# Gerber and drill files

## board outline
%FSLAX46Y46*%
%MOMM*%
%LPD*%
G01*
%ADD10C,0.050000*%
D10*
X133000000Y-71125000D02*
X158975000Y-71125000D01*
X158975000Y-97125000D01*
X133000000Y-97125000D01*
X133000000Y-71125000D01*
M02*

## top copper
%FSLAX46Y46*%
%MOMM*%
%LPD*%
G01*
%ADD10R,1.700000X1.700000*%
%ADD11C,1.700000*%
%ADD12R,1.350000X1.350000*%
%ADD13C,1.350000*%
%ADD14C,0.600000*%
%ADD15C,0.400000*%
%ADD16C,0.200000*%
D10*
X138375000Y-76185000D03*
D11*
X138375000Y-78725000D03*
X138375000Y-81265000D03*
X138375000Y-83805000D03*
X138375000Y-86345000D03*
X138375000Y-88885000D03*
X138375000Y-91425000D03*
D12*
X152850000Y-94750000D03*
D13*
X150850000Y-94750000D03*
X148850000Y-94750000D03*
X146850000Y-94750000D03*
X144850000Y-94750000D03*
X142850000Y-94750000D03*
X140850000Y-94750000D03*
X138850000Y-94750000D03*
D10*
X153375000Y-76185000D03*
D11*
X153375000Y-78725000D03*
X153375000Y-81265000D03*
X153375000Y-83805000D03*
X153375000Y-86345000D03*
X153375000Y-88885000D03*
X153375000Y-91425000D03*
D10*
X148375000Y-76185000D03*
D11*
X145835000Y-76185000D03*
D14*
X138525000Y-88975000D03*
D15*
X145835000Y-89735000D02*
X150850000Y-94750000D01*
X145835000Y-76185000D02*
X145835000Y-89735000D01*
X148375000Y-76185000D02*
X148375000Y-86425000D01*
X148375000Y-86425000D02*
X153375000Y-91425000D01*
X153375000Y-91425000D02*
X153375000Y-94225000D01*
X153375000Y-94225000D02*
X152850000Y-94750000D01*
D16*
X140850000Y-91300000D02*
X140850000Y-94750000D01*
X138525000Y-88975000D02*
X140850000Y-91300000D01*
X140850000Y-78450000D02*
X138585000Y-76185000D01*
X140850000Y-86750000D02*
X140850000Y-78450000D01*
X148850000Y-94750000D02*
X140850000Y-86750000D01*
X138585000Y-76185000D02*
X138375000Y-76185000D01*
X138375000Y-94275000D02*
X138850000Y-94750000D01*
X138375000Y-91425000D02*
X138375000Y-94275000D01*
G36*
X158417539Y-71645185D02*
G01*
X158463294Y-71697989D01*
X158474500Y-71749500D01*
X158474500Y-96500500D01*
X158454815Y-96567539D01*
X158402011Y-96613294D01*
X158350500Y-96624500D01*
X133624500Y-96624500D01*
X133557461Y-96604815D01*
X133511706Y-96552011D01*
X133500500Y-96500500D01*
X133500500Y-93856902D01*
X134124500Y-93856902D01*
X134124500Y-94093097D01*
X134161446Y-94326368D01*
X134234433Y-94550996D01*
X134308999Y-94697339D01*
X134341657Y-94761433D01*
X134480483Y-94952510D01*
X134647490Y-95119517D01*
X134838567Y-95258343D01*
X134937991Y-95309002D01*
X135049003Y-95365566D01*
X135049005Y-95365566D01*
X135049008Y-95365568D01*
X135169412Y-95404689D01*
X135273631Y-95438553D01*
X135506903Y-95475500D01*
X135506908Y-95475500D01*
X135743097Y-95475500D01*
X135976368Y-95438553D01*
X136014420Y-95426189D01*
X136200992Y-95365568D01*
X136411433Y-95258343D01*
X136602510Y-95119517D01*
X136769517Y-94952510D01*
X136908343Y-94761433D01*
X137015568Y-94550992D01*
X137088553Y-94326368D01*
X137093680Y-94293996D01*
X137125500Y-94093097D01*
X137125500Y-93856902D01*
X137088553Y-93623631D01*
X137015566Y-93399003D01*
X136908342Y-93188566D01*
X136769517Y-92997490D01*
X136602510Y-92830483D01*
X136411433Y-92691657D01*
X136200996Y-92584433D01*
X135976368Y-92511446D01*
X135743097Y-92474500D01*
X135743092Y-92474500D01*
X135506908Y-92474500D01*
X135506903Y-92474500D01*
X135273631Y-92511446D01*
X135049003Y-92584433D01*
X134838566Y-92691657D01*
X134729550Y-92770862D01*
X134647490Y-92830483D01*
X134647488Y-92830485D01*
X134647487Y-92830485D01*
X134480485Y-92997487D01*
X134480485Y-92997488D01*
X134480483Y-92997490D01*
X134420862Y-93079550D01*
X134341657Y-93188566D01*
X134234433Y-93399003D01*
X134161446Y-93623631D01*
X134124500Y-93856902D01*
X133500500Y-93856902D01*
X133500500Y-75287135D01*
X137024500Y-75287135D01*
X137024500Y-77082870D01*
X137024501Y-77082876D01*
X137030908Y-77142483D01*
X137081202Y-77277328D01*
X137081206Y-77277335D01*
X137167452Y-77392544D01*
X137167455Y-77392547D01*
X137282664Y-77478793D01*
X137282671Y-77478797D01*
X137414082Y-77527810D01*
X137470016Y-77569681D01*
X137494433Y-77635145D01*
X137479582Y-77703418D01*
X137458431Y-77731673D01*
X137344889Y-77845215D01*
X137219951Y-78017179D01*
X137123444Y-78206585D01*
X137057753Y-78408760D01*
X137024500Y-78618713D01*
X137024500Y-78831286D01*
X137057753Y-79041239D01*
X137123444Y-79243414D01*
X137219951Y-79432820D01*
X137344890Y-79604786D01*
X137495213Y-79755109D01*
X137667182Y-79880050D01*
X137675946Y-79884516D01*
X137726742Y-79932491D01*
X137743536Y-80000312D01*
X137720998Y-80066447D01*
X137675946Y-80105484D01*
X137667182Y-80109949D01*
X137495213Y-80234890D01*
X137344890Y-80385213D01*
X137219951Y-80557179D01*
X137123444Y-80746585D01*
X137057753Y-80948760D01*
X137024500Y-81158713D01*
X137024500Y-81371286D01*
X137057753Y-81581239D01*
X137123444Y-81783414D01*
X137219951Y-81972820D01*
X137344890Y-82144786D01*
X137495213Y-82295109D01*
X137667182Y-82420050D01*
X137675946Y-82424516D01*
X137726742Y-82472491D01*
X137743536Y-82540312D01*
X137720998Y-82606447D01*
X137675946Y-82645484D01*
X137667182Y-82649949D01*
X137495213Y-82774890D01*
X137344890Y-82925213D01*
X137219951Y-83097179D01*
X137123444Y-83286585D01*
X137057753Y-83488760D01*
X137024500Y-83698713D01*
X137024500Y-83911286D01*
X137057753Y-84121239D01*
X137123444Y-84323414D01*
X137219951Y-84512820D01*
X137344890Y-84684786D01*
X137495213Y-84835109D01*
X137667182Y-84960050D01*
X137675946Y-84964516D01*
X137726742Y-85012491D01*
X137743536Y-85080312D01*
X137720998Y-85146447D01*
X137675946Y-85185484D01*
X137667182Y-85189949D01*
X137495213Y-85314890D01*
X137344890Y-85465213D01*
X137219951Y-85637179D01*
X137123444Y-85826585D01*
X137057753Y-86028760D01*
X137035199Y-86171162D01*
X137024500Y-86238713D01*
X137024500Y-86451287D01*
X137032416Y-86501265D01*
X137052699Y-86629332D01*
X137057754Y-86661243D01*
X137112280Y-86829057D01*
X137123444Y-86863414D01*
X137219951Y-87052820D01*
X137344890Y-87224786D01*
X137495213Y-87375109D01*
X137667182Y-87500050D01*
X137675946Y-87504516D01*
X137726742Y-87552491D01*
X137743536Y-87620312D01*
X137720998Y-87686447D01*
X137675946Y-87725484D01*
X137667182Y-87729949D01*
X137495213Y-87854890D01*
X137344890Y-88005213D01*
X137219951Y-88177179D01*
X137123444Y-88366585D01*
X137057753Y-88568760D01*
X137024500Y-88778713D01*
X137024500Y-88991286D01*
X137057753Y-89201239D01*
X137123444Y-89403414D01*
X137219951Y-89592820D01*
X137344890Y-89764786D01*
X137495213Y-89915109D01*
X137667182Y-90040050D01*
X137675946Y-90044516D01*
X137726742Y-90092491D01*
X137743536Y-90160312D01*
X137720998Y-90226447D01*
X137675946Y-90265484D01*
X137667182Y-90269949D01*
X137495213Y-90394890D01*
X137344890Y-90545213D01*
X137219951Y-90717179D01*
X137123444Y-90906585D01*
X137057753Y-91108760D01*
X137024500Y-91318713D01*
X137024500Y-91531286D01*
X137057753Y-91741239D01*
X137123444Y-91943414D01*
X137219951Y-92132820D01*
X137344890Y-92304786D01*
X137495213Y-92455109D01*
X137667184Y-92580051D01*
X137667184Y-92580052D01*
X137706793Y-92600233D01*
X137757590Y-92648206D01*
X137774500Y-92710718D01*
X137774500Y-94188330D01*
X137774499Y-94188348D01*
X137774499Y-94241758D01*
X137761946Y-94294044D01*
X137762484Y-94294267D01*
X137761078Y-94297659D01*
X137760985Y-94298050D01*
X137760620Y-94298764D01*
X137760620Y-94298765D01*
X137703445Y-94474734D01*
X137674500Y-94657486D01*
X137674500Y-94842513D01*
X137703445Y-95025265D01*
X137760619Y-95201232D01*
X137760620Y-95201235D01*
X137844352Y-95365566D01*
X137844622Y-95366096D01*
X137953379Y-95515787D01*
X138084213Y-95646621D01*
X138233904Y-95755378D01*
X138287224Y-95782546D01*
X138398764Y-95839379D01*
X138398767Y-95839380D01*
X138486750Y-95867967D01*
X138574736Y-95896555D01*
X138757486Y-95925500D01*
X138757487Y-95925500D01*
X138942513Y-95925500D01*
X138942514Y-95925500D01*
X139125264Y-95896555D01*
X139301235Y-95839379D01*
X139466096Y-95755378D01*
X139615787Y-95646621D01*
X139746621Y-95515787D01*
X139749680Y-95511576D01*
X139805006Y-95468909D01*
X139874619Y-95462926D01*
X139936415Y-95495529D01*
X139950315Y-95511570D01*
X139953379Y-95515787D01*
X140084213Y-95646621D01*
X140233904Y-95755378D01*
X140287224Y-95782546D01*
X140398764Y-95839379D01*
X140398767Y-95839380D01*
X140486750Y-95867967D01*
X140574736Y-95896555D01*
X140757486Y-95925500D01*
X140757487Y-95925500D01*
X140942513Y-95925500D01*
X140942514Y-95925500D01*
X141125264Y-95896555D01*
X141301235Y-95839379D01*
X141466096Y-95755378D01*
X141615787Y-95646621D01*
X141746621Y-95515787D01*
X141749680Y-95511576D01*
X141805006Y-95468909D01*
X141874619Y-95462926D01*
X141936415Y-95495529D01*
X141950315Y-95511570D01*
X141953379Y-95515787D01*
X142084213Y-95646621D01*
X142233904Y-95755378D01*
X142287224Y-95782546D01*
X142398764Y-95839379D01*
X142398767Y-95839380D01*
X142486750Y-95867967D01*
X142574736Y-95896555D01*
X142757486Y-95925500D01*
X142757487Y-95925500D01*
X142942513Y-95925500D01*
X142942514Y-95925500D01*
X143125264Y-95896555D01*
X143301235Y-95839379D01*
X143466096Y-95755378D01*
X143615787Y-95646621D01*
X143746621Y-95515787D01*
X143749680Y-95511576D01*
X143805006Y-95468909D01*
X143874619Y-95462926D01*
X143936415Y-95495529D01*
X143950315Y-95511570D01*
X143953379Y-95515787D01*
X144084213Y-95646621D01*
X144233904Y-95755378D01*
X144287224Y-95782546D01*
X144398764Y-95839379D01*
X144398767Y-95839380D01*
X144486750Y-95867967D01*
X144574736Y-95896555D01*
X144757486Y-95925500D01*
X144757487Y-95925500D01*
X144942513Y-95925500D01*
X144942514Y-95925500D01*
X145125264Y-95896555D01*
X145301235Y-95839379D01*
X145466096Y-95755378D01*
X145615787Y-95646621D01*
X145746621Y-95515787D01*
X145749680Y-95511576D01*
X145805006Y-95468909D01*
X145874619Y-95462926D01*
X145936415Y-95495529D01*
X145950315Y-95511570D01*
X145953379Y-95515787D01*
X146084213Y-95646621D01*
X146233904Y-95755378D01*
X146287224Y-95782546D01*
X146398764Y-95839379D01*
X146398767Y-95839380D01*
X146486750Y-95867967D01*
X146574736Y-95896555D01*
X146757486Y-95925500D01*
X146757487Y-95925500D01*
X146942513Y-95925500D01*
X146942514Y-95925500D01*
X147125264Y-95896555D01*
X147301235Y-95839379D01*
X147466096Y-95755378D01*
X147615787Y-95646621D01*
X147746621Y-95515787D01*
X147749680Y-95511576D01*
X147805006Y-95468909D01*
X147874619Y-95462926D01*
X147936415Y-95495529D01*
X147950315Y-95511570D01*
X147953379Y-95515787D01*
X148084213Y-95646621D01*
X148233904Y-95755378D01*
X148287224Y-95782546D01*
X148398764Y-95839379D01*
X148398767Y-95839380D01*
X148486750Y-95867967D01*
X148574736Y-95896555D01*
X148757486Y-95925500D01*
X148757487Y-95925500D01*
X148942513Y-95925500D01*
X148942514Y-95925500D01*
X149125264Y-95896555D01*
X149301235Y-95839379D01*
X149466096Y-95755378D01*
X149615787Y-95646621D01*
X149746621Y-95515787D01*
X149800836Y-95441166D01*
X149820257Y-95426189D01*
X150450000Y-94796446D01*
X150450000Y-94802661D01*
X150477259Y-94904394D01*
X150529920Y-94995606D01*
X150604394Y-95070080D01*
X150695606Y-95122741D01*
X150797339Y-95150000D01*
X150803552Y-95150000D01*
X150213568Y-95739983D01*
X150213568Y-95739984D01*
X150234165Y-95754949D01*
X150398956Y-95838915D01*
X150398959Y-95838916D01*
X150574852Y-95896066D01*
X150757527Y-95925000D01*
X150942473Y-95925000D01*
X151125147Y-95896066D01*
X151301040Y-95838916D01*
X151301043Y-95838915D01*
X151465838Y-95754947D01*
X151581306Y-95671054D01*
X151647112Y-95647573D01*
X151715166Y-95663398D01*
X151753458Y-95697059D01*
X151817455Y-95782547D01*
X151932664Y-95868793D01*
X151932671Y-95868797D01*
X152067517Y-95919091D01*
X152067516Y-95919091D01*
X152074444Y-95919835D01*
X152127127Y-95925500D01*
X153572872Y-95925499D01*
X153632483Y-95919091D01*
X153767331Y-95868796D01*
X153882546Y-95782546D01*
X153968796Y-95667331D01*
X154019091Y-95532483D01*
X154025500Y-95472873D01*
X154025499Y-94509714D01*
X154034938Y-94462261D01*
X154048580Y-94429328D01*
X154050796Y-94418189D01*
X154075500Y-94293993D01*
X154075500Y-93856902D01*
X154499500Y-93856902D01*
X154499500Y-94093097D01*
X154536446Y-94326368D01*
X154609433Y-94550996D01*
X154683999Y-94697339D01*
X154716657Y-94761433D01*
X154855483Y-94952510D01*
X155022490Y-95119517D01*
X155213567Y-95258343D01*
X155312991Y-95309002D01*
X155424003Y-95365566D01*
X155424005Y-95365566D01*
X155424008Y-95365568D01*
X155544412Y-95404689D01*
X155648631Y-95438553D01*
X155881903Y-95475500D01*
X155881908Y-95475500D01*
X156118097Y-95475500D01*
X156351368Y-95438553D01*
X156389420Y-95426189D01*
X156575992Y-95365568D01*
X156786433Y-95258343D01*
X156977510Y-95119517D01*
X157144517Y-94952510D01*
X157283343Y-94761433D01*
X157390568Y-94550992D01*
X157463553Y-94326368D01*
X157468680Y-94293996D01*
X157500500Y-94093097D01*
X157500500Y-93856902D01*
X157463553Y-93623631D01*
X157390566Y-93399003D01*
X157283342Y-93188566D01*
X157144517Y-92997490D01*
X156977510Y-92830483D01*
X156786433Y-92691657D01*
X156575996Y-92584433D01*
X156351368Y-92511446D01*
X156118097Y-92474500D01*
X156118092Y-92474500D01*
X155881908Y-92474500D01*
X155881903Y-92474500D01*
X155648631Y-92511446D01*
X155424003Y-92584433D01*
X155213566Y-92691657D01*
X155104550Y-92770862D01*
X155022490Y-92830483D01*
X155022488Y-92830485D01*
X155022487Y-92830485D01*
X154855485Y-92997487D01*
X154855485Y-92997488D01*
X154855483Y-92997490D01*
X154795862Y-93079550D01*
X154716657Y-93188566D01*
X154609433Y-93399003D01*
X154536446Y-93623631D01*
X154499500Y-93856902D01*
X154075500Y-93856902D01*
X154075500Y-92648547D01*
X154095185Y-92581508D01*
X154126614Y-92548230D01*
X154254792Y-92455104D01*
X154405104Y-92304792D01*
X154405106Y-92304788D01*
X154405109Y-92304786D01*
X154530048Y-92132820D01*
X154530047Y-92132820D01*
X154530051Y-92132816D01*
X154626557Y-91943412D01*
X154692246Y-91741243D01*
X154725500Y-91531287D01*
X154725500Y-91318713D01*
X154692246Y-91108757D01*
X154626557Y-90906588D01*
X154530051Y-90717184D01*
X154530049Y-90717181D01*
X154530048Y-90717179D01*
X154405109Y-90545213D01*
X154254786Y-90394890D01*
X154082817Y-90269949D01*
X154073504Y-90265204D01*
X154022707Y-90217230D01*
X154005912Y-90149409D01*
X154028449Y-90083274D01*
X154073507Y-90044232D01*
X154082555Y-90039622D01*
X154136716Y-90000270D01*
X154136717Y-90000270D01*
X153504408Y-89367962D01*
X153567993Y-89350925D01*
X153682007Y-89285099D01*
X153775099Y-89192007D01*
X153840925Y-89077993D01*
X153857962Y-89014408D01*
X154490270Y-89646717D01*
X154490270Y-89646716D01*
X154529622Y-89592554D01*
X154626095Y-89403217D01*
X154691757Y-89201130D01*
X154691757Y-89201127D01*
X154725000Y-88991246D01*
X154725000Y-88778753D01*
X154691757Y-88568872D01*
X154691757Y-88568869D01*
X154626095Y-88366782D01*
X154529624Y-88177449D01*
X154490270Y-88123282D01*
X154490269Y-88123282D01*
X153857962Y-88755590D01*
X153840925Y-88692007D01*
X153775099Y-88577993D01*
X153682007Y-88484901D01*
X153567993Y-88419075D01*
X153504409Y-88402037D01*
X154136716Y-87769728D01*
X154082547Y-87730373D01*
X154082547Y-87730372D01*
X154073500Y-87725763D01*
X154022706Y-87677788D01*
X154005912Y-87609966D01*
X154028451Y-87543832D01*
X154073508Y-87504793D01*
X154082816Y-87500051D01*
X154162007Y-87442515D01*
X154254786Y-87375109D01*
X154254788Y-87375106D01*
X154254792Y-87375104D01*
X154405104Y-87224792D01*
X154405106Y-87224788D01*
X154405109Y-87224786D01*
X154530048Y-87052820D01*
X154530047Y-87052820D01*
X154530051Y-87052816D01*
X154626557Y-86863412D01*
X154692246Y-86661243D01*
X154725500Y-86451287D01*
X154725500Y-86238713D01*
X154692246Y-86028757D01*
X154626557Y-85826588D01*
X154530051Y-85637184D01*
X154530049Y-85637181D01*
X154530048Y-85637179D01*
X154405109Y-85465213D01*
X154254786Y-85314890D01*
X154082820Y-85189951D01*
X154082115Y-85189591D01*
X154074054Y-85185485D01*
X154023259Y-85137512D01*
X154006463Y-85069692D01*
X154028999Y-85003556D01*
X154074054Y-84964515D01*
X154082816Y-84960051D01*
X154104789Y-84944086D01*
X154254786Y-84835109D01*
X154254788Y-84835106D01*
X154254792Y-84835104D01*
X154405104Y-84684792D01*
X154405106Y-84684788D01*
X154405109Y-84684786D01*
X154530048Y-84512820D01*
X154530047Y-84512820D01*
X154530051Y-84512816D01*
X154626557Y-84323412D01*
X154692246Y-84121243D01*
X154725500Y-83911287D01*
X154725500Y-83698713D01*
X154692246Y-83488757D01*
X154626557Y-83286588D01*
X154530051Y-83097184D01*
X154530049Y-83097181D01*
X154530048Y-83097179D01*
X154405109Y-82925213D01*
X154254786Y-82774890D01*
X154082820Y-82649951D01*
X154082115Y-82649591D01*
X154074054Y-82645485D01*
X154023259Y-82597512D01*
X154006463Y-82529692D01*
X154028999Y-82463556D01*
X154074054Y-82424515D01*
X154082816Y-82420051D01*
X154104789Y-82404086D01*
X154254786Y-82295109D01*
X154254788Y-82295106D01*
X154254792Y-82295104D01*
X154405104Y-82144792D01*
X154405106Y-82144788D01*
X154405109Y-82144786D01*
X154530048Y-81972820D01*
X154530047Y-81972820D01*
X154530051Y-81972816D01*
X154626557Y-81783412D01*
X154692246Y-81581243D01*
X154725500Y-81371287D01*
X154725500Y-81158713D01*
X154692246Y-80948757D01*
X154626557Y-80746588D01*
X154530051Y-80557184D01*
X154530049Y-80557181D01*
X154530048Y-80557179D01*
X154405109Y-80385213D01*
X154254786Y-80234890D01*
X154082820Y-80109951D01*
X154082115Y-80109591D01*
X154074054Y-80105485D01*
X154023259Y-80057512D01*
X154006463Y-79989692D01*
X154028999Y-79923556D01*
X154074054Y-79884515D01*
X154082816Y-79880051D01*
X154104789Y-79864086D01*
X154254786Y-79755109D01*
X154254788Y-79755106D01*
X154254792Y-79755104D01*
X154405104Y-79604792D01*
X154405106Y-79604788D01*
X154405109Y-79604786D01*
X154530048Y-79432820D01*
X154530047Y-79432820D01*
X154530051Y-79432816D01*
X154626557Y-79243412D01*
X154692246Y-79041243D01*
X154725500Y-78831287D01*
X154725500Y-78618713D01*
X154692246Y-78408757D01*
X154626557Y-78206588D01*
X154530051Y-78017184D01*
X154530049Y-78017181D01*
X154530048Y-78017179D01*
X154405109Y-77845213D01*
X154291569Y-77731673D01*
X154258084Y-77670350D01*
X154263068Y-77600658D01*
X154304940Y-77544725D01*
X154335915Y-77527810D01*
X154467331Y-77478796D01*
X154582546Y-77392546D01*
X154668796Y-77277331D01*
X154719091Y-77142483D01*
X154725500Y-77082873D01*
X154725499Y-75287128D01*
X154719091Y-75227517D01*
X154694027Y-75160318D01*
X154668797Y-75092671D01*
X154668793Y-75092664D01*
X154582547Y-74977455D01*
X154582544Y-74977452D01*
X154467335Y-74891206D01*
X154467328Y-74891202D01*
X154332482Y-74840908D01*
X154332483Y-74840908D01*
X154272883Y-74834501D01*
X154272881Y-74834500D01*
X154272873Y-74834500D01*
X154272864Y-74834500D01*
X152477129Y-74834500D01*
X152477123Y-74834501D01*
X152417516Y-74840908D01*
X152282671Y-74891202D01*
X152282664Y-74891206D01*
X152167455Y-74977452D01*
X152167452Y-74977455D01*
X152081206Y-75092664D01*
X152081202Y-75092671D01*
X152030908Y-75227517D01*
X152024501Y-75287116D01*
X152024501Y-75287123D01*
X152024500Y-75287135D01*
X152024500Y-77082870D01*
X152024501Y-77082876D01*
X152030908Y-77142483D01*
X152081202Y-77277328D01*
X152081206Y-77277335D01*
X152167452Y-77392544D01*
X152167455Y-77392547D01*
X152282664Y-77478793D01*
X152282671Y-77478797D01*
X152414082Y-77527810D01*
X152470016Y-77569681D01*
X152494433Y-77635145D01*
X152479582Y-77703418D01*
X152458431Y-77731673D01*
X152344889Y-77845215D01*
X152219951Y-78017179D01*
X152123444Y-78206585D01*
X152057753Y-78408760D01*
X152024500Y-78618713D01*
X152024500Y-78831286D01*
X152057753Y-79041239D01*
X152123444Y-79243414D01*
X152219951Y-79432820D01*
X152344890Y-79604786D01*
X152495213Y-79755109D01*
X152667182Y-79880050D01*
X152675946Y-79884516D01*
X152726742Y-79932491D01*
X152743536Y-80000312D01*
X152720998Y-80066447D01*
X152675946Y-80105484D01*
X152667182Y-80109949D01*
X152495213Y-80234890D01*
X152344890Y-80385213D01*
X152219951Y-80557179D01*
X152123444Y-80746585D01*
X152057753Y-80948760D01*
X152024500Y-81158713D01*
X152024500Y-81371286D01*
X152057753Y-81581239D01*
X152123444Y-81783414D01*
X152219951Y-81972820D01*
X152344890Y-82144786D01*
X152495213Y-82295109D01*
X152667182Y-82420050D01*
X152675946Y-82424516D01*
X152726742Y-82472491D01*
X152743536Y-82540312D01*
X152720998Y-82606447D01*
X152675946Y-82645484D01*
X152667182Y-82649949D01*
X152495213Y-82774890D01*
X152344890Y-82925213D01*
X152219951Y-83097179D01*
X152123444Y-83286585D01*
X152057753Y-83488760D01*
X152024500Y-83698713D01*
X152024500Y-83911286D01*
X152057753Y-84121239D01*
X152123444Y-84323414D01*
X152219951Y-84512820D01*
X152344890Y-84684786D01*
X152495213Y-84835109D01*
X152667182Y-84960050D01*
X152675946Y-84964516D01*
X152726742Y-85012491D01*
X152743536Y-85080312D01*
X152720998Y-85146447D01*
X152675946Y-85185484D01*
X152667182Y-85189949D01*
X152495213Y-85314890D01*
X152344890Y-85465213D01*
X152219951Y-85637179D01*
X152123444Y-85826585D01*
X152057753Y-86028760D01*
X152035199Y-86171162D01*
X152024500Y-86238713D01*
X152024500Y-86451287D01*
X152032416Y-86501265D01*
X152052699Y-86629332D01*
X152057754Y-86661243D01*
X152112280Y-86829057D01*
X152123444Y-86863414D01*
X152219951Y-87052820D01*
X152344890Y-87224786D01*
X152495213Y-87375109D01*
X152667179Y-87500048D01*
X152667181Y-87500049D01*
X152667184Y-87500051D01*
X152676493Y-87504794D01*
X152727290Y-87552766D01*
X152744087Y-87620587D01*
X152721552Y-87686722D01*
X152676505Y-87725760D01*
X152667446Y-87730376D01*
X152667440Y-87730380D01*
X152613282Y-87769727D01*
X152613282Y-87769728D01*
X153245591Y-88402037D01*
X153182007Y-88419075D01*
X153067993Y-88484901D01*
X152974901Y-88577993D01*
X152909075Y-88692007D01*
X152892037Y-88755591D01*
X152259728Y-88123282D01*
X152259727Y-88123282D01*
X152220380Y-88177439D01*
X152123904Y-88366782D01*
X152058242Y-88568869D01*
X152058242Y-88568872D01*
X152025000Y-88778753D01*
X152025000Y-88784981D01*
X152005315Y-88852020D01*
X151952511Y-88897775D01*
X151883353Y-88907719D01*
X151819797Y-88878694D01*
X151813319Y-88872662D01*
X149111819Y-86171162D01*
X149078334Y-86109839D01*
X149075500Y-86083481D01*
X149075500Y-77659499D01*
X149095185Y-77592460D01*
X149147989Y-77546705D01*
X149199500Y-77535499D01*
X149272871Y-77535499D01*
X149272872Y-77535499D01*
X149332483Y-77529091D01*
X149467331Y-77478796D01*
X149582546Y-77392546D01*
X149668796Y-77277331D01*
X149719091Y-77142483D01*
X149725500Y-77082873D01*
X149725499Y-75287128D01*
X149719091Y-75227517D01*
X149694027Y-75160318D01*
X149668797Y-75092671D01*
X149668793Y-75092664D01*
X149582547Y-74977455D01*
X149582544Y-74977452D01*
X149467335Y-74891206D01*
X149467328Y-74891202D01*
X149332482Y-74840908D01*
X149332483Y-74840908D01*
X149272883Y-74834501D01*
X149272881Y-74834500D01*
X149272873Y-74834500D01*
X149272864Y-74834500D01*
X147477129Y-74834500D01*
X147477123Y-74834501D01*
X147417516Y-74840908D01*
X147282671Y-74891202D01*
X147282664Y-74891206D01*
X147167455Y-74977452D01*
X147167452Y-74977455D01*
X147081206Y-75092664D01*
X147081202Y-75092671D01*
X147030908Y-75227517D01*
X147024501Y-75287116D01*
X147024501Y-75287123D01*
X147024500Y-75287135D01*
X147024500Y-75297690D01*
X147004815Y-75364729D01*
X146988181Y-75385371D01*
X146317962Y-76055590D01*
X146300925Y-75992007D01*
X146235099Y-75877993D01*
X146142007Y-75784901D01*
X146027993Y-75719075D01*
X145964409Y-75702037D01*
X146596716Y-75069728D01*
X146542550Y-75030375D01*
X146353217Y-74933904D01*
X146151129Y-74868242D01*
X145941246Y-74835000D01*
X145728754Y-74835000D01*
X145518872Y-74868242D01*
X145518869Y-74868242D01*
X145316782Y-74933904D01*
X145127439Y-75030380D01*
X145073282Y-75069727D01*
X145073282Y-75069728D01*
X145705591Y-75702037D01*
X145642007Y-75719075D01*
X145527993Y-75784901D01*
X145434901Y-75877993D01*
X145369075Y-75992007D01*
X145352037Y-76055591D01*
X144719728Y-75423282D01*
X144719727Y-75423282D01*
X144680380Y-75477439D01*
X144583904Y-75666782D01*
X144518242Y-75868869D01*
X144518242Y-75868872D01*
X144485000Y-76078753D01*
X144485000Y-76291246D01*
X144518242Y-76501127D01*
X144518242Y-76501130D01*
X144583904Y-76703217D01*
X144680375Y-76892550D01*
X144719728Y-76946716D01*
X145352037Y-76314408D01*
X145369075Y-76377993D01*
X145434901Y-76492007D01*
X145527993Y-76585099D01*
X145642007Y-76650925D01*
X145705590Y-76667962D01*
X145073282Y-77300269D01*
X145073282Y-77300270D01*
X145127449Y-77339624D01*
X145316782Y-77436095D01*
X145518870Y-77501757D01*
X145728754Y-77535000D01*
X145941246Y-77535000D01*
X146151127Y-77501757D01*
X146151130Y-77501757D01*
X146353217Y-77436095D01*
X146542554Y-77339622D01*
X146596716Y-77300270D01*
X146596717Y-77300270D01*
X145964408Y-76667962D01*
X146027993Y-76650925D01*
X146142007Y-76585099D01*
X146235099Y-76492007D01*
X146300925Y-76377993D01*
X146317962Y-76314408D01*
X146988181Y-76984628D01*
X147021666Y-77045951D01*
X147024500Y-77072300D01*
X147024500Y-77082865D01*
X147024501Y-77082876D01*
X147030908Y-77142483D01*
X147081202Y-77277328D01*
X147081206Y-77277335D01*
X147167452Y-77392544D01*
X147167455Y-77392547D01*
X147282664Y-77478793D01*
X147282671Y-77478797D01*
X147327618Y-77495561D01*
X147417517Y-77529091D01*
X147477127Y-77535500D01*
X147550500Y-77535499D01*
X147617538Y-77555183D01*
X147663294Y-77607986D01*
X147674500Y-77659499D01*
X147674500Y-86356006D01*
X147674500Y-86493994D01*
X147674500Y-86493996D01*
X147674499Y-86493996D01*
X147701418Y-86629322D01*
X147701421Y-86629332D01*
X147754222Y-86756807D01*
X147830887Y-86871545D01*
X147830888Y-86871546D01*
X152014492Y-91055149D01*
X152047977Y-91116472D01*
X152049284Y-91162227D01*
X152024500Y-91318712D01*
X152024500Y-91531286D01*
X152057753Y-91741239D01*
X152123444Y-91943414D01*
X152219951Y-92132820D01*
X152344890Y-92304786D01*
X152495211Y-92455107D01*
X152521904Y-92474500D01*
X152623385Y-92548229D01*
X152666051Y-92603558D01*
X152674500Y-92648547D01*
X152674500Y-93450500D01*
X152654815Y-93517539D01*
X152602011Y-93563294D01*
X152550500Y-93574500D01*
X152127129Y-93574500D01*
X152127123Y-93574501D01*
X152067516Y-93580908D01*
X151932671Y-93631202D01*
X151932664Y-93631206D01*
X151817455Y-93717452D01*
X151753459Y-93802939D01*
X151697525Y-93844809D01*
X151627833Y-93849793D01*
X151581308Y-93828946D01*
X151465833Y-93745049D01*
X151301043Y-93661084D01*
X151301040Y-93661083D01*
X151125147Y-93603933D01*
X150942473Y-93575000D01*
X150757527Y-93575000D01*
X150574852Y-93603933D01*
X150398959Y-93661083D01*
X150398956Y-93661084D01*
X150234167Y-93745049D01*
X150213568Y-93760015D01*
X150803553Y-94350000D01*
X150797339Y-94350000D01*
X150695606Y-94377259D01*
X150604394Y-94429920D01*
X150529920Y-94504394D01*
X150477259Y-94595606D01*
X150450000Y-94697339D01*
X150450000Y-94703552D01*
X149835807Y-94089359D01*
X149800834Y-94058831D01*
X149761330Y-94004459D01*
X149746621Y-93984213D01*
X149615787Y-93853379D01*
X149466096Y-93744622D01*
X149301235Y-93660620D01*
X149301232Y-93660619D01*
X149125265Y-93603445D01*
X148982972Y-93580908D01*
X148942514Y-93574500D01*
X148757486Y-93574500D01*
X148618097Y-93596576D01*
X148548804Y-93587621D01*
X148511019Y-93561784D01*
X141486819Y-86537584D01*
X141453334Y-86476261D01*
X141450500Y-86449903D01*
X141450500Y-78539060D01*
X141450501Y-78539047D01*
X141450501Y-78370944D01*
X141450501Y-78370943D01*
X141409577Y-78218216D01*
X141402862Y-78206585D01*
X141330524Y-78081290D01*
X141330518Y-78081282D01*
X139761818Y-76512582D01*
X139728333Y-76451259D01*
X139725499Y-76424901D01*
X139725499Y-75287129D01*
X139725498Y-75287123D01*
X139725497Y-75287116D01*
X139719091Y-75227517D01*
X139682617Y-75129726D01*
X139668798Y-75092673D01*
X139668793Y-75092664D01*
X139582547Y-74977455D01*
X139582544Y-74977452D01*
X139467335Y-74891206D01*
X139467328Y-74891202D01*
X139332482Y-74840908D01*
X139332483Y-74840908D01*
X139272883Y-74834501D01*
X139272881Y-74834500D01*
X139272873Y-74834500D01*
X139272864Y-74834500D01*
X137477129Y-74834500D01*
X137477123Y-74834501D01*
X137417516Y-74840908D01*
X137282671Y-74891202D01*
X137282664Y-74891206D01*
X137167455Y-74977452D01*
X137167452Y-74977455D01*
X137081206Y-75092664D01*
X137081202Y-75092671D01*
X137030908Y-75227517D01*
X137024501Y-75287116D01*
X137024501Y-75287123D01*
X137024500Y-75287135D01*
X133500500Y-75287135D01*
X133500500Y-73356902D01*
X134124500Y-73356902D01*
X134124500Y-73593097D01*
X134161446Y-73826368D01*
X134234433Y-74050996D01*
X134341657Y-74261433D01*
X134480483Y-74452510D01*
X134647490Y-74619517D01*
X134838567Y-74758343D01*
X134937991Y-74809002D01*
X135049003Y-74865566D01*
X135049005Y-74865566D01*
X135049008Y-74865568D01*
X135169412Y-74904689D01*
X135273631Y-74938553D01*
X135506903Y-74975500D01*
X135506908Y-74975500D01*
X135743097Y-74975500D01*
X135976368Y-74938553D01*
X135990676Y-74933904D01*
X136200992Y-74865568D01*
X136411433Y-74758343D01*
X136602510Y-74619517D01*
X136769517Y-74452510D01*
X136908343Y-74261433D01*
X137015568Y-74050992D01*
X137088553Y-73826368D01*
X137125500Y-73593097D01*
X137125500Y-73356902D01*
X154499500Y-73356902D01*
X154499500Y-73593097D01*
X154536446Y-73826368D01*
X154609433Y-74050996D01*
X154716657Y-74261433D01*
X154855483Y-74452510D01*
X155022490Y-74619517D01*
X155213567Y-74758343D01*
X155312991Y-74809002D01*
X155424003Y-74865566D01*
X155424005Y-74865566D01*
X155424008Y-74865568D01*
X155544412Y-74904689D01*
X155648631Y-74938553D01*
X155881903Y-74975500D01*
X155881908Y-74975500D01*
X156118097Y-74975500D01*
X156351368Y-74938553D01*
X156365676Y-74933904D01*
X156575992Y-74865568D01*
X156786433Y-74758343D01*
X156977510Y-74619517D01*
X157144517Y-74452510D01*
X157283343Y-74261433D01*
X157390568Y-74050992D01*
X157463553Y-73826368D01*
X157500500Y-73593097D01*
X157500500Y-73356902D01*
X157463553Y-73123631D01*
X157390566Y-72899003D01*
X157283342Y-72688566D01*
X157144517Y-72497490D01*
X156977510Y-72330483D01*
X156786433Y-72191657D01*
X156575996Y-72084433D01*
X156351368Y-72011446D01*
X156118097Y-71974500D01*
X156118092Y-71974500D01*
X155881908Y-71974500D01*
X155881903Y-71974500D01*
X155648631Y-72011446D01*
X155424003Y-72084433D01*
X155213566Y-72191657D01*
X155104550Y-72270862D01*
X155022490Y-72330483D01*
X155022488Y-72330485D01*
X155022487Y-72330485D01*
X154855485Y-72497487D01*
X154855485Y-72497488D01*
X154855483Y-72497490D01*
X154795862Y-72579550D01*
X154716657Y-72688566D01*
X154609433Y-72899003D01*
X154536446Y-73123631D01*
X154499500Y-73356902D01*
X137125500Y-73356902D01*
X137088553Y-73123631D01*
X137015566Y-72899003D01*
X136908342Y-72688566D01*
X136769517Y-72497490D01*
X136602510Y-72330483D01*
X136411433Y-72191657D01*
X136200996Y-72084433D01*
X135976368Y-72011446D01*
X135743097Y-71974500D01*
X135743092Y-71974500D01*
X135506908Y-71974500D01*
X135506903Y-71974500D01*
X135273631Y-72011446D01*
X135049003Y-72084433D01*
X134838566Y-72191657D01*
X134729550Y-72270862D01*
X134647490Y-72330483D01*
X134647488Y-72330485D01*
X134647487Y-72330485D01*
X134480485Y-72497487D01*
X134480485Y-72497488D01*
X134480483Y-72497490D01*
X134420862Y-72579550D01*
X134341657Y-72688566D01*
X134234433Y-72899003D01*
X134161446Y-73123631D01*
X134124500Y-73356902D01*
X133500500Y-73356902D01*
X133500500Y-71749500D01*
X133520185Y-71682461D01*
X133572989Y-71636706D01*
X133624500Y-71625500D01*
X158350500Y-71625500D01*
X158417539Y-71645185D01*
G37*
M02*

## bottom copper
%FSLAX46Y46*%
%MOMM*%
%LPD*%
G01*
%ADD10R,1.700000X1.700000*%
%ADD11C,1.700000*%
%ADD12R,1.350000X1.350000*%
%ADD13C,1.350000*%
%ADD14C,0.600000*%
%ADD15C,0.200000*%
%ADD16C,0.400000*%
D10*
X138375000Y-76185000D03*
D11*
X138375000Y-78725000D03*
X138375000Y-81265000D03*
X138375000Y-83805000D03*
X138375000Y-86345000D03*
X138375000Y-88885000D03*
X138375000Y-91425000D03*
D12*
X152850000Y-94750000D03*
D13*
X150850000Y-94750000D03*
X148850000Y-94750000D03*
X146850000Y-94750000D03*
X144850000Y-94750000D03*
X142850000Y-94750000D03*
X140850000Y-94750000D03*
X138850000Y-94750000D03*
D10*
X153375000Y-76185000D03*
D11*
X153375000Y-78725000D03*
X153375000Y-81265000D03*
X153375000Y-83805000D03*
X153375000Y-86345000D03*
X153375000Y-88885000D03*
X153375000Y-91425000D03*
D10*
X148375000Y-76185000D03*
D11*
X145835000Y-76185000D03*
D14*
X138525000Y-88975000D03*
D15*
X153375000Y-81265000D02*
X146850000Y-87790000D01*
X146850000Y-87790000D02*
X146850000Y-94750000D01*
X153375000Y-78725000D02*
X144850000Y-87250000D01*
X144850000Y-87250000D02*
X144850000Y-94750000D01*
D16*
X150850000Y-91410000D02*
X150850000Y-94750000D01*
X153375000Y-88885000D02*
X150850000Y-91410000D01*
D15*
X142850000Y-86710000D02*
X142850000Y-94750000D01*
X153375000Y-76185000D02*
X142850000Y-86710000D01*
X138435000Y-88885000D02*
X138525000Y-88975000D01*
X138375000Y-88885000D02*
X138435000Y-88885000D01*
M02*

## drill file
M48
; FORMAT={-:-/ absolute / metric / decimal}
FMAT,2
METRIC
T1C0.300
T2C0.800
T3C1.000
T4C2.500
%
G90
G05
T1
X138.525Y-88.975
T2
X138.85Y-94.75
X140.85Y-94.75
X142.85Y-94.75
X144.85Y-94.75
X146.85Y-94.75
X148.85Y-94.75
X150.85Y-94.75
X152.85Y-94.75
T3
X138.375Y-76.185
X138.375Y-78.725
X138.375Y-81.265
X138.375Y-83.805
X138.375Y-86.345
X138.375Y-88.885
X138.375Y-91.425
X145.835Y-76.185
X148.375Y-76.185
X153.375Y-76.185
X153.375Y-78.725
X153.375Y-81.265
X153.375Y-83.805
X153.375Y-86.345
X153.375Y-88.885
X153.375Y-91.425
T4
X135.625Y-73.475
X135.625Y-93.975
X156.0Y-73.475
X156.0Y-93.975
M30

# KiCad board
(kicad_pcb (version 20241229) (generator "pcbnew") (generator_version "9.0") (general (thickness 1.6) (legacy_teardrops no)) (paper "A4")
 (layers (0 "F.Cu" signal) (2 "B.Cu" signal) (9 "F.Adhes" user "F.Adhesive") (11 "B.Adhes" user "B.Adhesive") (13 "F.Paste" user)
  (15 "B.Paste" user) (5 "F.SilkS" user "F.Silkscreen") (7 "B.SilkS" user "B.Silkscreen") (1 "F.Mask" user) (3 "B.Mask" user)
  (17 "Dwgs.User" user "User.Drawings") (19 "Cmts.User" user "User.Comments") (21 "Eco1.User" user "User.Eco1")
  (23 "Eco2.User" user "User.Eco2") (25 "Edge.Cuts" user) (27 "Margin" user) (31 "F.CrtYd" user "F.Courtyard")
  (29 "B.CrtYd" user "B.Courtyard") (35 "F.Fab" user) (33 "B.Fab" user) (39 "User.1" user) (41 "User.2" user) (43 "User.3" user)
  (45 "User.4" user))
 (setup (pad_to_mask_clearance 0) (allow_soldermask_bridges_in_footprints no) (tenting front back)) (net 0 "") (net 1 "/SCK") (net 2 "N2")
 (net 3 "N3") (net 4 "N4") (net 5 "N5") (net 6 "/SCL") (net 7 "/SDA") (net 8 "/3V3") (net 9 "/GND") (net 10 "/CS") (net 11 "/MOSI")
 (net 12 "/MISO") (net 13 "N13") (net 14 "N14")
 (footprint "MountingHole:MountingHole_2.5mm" (layer "F.Cu") (at 135.625 73.475)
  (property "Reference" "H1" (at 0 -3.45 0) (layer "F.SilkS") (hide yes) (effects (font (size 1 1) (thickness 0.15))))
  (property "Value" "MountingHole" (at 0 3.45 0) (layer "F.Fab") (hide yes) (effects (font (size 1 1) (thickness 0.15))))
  (pad "" np_thru_hole circle (at 0 0) (size 2.5 2.5) (drill 2.5) (layers "*.Cu" "*.Mask")))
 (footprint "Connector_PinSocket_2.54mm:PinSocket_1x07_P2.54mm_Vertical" (layer "F.Cu") (at 138.375 76.185)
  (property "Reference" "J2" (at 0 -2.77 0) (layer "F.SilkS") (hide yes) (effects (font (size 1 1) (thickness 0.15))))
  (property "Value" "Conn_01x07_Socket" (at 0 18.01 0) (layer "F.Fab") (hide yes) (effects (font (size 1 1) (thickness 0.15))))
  (pad "1" thru_hole rect (at 0 0) (size 1.7 1.7) (drill 1) (layers "*.Cu" "*.Mask") (remove_unused_layers no) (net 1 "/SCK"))
  (pad "2" thru_hole circle (at 0 2.54) (size 1.7 1.7) (drill 1) (layers "*.Cu" "*.Mask") (remove_unused_layers no) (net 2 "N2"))
  (pad "3" thru_hole circle (at 0 5.08) (size 1.7 1.7) (drill 1) (layers "*.Cu" "*.Mask") (remove_unused_layers no) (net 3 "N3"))
  (pad "4" thru_hole circle (at 0 7.62) (size 1.7 1.7) (drill 1) (layers "*.Cu" "*.Mask") (remove_unused_layers no) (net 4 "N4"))
  (pad "5" thru_hole circle (at 0 10.16) (size 1.7 1.7) (drill 1) (layers "*.Cu" "*.Mask") (remove_unused_layers no) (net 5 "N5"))
  (pad "6" thru_hole circle (at 0 12.7) (size 1.7 1.7) (drill 1) (layers "*.Cu" "*.Mask") (remove_unused_layers no) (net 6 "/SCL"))
  (pad "7" thru_hole circle (at 0 15.24) (size 1.7 1.7) (drill 1) (layers "*.Cu" "*.Mask") (remove_unused_layers no) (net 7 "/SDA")))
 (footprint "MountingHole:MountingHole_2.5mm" (layer "F.Cu") (at 156.125 93.975)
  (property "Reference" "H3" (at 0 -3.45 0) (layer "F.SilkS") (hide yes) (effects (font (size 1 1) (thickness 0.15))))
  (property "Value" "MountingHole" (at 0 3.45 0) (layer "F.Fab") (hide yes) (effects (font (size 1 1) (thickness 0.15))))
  (pad "" np_thru_hole circle (at -0.125 0) (size 2.5 2.5) (drill 2.5) (layers "*.Cu" "*.Mask")))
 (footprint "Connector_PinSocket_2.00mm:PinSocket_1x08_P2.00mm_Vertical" (layer "F.Cu") (at 152.85 94.75 -90)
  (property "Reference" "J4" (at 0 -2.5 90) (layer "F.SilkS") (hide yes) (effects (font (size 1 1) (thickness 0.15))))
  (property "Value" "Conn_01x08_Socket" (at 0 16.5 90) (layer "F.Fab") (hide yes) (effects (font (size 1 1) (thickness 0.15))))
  (pad "1" thru_hole rect (at 0 0 270) (size 1.35 1.35) (drill 0.8) (layers "*.Cu" "*.Mask") (remove_unused_layers no) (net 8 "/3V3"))
  (pad "2" thru_hole circle (at 0 2 270) (size 1.35 1.35) (drill 0.8) (layers "*.Cu" "*.Mask") (remove_unused_layers no) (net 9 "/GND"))
  (pad "3" thru_hole circle (at 0 4 270) (size 1.35 1.35) (drill 0.8) (layers "*.Cu" "*.Mask") (remove_unused_layers no) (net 1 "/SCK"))
  (pad "4" thru_hole circle (at 0 6 270) (size 1.35 1.35) (drill 0.8) (layers "*.Cu" "*.Mask") (remove_unused_layers no) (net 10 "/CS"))
  (pad "5" thru_hole circle (at 0 8 270) (size 1.35 1.35) (drill 0.8) (layers "*.Cu" "*.Mask") (remove_unused_layers no) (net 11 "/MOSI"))
  (pad "6" thru_hole circle (at 0 10 270) (size 1.35 1.35) (drill 0.8) (layers "*.Cu" "*.Mask") (remove_unused_layers no) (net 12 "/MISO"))
  (pad "7" thru_hole circle (at 0 12 270) (size 1.35 1.35) (drill 0.8) (layers "*.Cu" "*.Mask") (remove_unused_layers no) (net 6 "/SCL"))
  (pad "8" thru_hole circle (at 0 14 270) (size 1.35 1.35) (drill 0.8) (layers "*.Cu" "*.Mask") (remove_unused_layers no) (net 7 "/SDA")))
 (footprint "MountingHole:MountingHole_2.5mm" (layer "F.Cu") (at 156.125 73.475)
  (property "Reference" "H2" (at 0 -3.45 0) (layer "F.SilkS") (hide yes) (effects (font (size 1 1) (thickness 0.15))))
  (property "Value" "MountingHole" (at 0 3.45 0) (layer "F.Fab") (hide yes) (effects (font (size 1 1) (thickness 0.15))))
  (pad "" np_thru_hole circle (at -0.125 0) (size 2.5 2.5) (drill 2.5) (layers "*.Cu" "*.Mask")))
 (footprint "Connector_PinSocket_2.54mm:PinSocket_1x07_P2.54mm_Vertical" (layer "F.Cu") (at 153.375 76.185)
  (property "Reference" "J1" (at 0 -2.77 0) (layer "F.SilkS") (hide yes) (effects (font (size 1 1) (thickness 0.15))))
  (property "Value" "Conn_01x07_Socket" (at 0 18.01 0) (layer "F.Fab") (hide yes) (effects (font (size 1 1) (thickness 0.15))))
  (pad "1" thru_hole rect (at 0 0) (size 1.7 1.7) (drill 1) (layers "*.Cu" "*.Mask") (remove_unused_layers no) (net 12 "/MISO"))
  (pad "2" thru_hole circle (at 0 2.54) (size 1.7 1.7) (drill 1) (layers "*.Cu" "*.Mask") (remove_unused_layers no) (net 11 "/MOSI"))
  (pad "3" thru_hole circle (at 0 5.08) (size 1.7 1.7) (drill 1) (layers "*.Cu" "*.Mask") (remove_unused_layers no) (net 10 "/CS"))
  (pad "4" thru_hole circle (at 0 7.62) (size 1.7 1.7) (drill 1) (layers "*.Cu" "*.Mask") (remove_unused_layers no) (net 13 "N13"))
  (pad "5" thru_hole circle (at 0 10.16) (size 1.7 1.7) (drill 1) (layers "*.Cu" "*.Mask") (remove_unused_layers no) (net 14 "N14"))
  (pad "6" thru_hole circle (at 0 12.7) (size 1.7 1.7) (drill 1) (layers "*.Cu" "*.Mask") (remove_unused_layers no) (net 9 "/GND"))
  (pad "7" thru_hole circle (at 0 15.24) (size 1.7 1.7) (drill 1) (layers "*.Cu" "*.Mask") (remove_unused_layers no) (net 8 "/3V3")))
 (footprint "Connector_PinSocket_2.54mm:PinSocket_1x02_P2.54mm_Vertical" (layer "F.Cu") (at 148.375 76.185 -90)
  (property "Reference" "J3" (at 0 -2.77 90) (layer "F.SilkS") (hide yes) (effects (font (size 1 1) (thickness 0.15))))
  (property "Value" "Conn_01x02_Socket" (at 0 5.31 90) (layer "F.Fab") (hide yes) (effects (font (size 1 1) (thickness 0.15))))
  (pad "1" thru_hole rect (at 0 0 270) (size 1.7 1.7) (drill 1) (layers "*.Cu" "*.Mask") (remove_unused_layers no) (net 8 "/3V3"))
  (pad "2" thru_hole circle (at 0 2.54 270) (size 1.7 1.7) (drill 1) (layers "*.Cu" "*.Mask") (remove_unused_layers no) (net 9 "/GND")))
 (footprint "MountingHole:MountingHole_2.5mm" (layer "F.Cu") (at 135.625 93.975)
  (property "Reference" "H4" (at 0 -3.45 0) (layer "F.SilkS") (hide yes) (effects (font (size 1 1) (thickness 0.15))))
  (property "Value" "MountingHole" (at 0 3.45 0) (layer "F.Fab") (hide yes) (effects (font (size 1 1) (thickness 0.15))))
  (pad "" np_thru_hole circle (at 0 0) (size 2.5 2.5) (drill 2.5) (layers "*.Cu" "*.Mask")))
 (gr_rect (start 133 71.125) (end 158.975 97.125) (stroke (width 0.05) (type default)) (fill no) (layer "Edge.Cuts"))
 (segment (start 153.375 81.265) (end 146.85 87.79) (width 0.2) (layer "B.Cu") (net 10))
 (segment (start 146.85 87.79) (end 146.85 94.75) (width 0.2) (layer "B.Cu") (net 10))
 (segment (start 153.375 78.725) (end 144.85 87.25) (width 0.2) (layer "B.Cu") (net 11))
 (segment (start 144.85 87.25) (end 144.85 94.75) (width 0.2) (layer "B.Cu") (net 11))
 (segment (start 145.835 89.735) (end 150.85 94.75) (width 0.4) (layer "F.Cu") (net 9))
 (segment (start 145.835 76.185) (end 145.835 89.735) (width 0.4) (layer "F.Cu") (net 9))
 (segment (start 150.85 91.41) (end 150.85 94.75) (width 0.4) (layer "B.Cu") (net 9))
 (segment (start 153.375 88.885) (end 150.85 91.41) (width 0.4) (layer "B.Cu") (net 9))
 (segment (start 142.85 86.71) (end 142.85 94.75) (width 0.2) (layer "B.Cu") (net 12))
 (segment (start 153.375 76.185) (end 142.85 86.71) (width 0.2) (layer "B.Cu") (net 12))
 (segment (start 148.375 76.185) (end 148.375 86.425) (width 0.4) (layer "F.Cu") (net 8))
 (segment (start 148.375 86.425) (end 153.375 91.425) (width 0.4) (layer "F.Cu") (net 8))
 (segment (start 153.375 91.425) (end 153.375 94.225) (width 0.4) (layer "F.Cu") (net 8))
 (segment (start 153.375 94.225) (end 152.85 94.75) (width 0.4) (layer "F.Cu") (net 8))
 (segment (start 140.85 91.3) (end 140.85 94.75) (width 0.2) (layer "F.Cu") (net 6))
 (segment (start 138.525 88.975) (end 140.85 91.3) (width 0.2) (layer "F.Cu") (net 6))
 (via (at 138.525 88.975) (size 0.6) (drill 0.3) (layers "F.Cu" "B.Cu") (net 6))
 (segment (start 138.435 88.885) (end 138.525 88.975) (width 0.2) (layer "B.Cu") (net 6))
 (segment (start 138.375 88.885) (end 138.435 88.885) (width 0.2) (layer "B.Cu") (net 6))
 (segment (start 140.85 78.45) (end 138.585 76.185) (width 0.2) (layer "F.Cu") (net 1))
 (segment (start 140.85 86.75) (end 140.85 78.45) (width 0.2) (layer "F.Cu") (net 1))
 (segment (start 148.85 94.75) (end 140.85 86.75) (width 0.2) (layer "F.Cu") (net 1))
 (segment (start 138.585 76.185) (end 138.375 76.185) (width 0.2) (layer "F.Cu") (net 1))
 (segment (start 138.375 94.275) (end 138.85 94.75) (width 0.2) (layer "F.Cu") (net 7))
 (segment (start 138.375 91.425) (end 138.375 94.275) (width 0.2) (layer "F.Cu") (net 7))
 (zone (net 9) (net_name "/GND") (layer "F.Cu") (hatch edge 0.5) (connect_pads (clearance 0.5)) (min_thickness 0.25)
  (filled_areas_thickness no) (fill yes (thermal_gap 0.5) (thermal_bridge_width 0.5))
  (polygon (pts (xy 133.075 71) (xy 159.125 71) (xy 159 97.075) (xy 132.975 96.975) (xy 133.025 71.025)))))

